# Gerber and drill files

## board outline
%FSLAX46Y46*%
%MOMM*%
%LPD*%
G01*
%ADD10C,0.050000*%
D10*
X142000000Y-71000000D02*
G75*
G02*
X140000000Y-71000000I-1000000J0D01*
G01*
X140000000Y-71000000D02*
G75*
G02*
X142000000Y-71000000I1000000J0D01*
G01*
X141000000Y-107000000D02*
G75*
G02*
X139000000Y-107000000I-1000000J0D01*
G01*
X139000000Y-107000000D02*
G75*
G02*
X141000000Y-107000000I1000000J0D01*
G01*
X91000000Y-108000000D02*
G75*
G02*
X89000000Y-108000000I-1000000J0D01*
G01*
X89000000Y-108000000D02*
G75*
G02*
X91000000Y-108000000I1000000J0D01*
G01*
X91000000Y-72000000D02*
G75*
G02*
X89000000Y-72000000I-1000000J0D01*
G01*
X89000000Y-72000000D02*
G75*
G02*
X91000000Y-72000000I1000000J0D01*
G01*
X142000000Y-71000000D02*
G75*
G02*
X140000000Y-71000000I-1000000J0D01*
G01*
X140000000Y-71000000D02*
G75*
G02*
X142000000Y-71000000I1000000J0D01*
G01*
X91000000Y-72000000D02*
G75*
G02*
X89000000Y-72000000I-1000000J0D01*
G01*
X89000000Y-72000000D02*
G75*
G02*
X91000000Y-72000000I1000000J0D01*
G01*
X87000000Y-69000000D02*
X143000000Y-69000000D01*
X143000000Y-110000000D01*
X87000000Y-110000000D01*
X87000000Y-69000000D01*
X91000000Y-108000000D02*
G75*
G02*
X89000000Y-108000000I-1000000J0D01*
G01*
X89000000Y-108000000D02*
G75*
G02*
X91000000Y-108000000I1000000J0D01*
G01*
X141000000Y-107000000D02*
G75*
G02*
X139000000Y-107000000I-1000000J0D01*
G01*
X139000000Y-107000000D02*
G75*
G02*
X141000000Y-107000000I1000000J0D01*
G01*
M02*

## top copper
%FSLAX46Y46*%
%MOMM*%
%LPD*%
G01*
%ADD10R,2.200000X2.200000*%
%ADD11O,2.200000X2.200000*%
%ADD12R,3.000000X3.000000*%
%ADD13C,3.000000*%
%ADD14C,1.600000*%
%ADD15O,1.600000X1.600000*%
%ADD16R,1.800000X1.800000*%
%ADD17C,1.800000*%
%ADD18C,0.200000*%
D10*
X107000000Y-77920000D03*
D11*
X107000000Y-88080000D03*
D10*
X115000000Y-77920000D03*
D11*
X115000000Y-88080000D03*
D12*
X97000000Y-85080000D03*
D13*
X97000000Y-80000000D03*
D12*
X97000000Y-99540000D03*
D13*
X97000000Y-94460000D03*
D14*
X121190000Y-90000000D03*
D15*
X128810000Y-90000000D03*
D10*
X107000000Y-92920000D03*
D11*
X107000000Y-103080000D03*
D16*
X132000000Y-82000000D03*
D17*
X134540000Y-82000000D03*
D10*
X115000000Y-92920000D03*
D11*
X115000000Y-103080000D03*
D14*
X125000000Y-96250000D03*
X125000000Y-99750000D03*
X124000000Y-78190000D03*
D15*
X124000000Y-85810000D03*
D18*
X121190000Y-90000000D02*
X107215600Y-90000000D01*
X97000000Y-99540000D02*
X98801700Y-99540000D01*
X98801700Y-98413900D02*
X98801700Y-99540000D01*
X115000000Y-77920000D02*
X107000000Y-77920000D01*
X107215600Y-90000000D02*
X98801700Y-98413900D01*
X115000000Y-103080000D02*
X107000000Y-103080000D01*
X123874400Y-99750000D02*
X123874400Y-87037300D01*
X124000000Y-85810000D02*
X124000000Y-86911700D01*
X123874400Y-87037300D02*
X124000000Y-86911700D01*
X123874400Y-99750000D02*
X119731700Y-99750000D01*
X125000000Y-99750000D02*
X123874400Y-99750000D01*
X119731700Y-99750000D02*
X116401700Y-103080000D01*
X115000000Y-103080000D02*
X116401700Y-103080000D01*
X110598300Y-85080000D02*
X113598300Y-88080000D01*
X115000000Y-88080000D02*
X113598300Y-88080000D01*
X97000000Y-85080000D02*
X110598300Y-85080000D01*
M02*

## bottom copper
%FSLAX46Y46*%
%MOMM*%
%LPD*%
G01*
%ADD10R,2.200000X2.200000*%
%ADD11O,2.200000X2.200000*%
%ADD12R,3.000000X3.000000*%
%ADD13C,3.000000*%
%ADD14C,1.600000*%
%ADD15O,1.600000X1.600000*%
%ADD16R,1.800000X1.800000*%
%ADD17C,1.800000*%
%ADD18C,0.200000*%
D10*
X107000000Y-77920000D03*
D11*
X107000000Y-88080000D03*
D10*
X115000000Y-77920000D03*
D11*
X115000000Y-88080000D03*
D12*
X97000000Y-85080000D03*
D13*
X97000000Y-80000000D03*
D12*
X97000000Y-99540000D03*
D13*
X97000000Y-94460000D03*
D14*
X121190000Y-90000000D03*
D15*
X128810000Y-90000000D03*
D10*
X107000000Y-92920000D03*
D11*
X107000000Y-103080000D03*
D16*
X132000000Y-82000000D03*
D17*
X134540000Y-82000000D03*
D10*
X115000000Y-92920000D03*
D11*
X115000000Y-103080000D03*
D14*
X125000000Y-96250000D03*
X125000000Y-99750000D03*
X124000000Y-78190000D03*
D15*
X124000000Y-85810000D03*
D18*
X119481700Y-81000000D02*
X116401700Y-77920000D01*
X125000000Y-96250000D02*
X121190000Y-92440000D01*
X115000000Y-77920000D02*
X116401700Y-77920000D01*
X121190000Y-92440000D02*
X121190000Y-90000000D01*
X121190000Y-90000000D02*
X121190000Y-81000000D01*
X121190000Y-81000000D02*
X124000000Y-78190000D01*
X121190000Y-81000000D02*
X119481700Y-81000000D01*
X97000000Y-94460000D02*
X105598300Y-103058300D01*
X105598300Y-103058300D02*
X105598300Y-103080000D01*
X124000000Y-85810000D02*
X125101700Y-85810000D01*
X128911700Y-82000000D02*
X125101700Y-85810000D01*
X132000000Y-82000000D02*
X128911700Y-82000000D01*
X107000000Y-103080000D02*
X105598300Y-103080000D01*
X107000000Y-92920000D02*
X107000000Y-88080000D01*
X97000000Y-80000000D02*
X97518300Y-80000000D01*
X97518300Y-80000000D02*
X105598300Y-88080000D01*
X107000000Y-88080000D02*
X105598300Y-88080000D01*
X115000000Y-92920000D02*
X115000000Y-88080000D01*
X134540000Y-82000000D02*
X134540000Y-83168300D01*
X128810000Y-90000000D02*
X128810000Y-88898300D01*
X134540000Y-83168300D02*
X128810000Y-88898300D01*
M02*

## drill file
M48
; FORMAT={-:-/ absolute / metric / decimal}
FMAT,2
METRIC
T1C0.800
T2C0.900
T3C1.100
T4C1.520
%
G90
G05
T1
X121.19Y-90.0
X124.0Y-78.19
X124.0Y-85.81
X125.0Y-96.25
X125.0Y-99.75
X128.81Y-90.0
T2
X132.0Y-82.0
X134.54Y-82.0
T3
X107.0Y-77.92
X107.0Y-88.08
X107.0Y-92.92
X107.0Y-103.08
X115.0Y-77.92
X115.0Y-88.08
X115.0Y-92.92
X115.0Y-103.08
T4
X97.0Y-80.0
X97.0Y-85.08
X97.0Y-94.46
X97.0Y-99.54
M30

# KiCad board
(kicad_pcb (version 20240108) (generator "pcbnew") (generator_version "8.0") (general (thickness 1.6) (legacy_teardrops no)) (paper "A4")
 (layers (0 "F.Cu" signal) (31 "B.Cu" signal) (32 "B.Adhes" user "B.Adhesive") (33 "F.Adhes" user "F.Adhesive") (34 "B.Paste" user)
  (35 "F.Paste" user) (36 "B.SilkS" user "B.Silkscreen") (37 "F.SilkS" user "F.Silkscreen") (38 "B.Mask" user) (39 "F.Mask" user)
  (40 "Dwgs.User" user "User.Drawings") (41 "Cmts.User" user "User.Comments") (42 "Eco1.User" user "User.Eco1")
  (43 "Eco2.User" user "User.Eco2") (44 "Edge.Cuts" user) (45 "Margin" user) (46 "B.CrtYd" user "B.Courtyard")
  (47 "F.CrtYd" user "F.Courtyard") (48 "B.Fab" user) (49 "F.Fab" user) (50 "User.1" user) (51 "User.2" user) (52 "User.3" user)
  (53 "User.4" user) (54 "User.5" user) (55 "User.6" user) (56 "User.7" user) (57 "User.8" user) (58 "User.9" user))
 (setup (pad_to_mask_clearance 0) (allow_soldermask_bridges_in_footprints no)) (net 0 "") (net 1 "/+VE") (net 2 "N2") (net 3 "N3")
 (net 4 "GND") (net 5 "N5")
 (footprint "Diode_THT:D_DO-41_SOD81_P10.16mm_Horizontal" (layer "F.Cu") (at 107 77.92 -90)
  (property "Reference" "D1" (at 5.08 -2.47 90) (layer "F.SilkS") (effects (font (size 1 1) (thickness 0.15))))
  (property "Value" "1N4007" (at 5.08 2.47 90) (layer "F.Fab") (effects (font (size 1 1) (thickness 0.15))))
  (pad "1" thru_hole rect (at 0 0 270) (size 2.2 2.2) (drill 1.1) (layers "*.Cu" "*.Mask") (remove_unused_layers no) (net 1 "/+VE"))
  (pad "2" thru_hole oval (at 10.16 0 270) (size 2.2 2.2) (drill 1.1) (layers "*.Cu" "*.Mask") (remove_unused_layers no) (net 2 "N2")))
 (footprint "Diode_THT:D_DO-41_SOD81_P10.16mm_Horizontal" (layer "F.Cu") (at 115 77.92 -90)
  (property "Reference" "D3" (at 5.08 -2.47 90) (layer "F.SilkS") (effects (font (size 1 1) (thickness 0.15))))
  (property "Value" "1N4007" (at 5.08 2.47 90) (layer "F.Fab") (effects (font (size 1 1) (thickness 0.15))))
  (pad "1" thru_hole rect (at 0 0 270) (size 2.2 2.2) (drill 1.1) (layers "*.Cu" "*.Mask") (remove_unused_layers no) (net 1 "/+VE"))
  (pad "2" thru_hole oval (at 10.16 0 270) (size 2.2 2.2) (drill 1.1) (layers "*.Cu" "*.Mask") (remove_unused_layers no) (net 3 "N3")))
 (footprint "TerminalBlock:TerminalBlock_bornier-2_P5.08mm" (layer "F.Cu") (at 97 85.08 90)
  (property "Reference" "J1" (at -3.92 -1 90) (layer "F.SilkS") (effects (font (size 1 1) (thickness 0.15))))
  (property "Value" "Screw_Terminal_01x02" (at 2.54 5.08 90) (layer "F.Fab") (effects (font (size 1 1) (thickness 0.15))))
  (pad "1" thru_hole rect (at 0 0 90) (size 3 3) (drill 1.52) (layers "*.Cu" "*.Mask") (remove_unused_layers no) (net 3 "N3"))
  (pad "2" thru_hole circle (at 5.08 0 90) (size 3 3) (drill 1.52) (layers "*.Cu" "*.Mask") (remove_unused_layers no) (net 2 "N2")))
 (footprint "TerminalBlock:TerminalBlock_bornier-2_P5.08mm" (layer "F.Cu") (at 97 99.54 90)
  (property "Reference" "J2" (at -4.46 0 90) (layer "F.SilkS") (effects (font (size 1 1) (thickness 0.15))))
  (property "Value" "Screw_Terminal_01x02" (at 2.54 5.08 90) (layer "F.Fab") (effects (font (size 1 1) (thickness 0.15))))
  (pad "1" thru_hole rect (at 0 0 90) (size 3 3) (drill 1.52) (layers "*.Cu" "*.Mask") (remove_unused_layers no) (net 1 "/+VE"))
  (pad "2" thru_hole circle (at 5.08 0 90) (size 3 3) (drill 1.52) (layers "*.Cu" "*.Mask") (remove_unused_layers no) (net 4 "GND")))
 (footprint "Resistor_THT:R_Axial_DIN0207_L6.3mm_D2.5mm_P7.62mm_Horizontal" (layer "F.Cu") (at 121.19 90)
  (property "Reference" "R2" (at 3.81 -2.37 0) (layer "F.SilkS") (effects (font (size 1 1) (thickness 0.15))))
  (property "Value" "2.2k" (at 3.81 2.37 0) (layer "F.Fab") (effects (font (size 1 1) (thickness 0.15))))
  (pad "1" thru_hole circle (at 0 0) (size 1.6 1.6) (drill 0.8) (layers "*.Cu" "*.Mask") (remove_unused_layers no) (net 1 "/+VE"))
  (pad "2" thru_hole oval (at 7.62 0) (size 1.6 1.6) (drill 0.8) (layers "*.Cu" "*.Mask") (remove_unused_layers no) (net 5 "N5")))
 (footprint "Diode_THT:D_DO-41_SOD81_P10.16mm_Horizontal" (layer "F.Cu") (at 107 92.92 -90)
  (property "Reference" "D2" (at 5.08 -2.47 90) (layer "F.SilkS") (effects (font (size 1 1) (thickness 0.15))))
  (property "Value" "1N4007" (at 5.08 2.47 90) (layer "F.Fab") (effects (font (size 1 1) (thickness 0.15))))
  (pad "1" thru_hole rect (at 0 0 270) (size 2.2 2.2) (drill 1.1) (layers "*.Cu" "*.Mask") (remove_unused_layers no) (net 2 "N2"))
  (pad "2" thru_hole oval (at 10.16 0 270) (size 2.2 2.2) (drill 1.1) (layers "*.Cu" "*.Mask") (remove_unused_layers no) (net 4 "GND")))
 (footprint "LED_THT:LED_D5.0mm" (layer "F.Cu") (at 132 82)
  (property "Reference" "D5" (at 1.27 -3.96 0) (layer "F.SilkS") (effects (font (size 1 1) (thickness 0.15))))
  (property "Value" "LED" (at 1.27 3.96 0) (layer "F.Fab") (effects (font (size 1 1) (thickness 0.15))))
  (pad "1" thru_hole rect (at 0 0) (size 1.8 1.8) (drill 0.9) (layers "*.Cu" "*.Mask") (remove_unused_layers no) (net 4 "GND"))
  (pad "2" thru_hole circle (at 2.54 0) (size 1.8 1.8) (drill 0.9) (layers "*.Cu" "*.Mask") (remove_unused_layers no) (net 5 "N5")))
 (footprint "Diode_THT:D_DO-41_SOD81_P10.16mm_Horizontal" (layer "F.Cu") (at 115 92.92 -90)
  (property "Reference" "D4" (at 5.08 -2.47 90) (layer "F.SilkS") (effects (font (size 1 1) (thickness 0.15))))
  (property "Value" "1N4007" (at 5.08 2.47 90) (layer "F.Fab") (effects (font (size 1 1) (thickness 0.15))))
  (pad "1" thru_hole rect (at 0 0 270) (size 2.2 2.2) (drill 1.1) (layers "*.Cu" "*.Mask") (remove_unused_layers no) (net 3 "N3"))
  (pad "2" thru_hole oval (at 10.16 0 270) (size 2.2 2.2) (drill 1.1) (layers "*.Cu" "*.Mask") (remove_unused_layers no) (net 4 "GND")))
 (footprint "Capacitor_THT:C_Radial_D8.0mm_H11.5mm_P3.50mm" (layer "F.Cu") (at 125 96.25 -90)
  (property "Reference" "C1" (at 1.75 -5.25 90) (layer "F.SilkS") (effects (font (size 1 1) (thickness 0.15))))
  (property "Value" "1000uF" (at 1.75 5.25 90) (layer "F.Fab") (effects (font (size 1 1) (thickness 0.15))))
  (pad "1" thru_hole circle (at 0 0 270) (size 1.6 1.6) (drill 0.8) (layers "*.Cu" "*.Mask") (remove_unused_layers no) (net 1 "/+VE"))
  (pad "2" thru_hole circle (at 3.5 0 270) (size 1.6 1.6) (drill 0.8) (layers "*.Cu" "*.Mask") (remove_unused_layers no) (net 4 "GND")))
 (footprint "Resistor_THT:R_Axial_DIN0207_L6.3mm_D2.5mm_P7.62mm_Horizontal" (layer "F.Cu") (at 124 78.19 -90)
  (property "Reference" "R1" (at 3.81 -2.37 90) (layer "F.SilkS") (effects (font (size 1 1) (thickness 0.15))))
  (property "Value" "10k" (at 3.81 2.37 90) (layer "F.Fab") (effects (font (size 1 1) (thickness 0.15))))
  (pad "1" thru_hole circle (at 0 0 270) (size 1.6 1.6) (drill 0.8) (layers "*.Cu" "*.Mask") (remove_unused_layers no) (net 1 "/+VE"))
  (pad "2" thru_hole oval (at 7.62 0 270) (size 1.6 1.6) (drill 0.8) (layers "*.Cu" "*.Mask") (remove_unused_layers no) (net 4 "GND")))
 (gr_circle (center 141 71) (end 141 70) (stroke (width 0.05) (type default)) (fill none) (layer "Edge.Cuts"))
 (gr_circle (center 140 107) (end 140 106) (stroke (width 0.05) (type default)) (fill none) (layer "Edge.Cuts"))
 (gr_circle (center 90 108) (end 90 107) (stroke (width 0.05) (type default)) (fill none) (layer "Edge.Cuts"))
 (gr_circle (center 90 72) (end 90 71) (stroke (width 0.05) (type default)) (fill none) (layer "Edge.Cuts"))
 (gr_circle (center 141 71) (end 141 70) (stroke (width 0.05) (type default)) (fill none) (layer "Edge.Cuts"))
 (gr_circle (center 90 72) (end 90 71) (stroke (width 0.05) (type default)) (fill none) (layer "Edge.Cuts"))
 (gr_rect (start 87 69) (end 143 110) (stroke (width 0.05) (type default)) (fill none) (layer "Edge.Cuts"))
 (gr_circle (center 90 108) (end 90 107) (stroke (width 0.05) (type default)) (fill none) (layer "Edge.Cuts"))
 (gr_circle (center 140 107) (end 140 106) (stroke (width 0.05) (type default)) (fill none) (layer "Edge.Cuts"))
 (segment (start 121.19 90) (end 107.2156 90) (width 0.2) (layer "F.Cu") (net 1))
 (segment (start 97 99.54) (end 98.8017 99.54) (width 0.2) (layer "F.Cu") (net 1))
 (segment (start 98.8017 98.4139) (end 98.8017 99.54) (width 0.2) (layer "F.Cu") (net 1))
 (segment (start 115 77.92) (end 107 77.92) (width 0.2) (layer "F.Cu") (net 1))
 (segment (start 107.2156 90) (end 98.8017 98.4139) (width 0.2) (layer "F.Cu") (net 1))
 (segment (start 119.4817 81) (end 116.4017 77.92) (width 0.2) (layer "B.Cu") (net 1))
 (segment (start 125 96.25) (end 121.19 92.44) (width 0.2) (layer "B.Cu") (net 1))
 (segment (start 115 77.92) (end 116.4017 77.92) (width 0.2) (layer "B.Cu") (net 1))
 (segment (start 121.19 92.44) (end 121.19 90) (width 0.2) (layer "B.Cu") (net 1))
 (segment (start 121.19 90) (end 121.19 81) (width 0.2) (layer "B.Cu") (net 1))
 (segment (start 121.19 81) (end 124 78.19) (width 0.2) (layer "B.Cu") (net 1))
 (segment (start 121.19 81) (end 119.4817 81) (width 0.2) (layer "B.Cu") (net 1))
 (segment (start 115 103.08) (end 107 103.08) (width 0.2) (layer "F.Cu") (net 4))
 (segment (start 123.8744 99.75) (end 123.8744 87.0373) (width 0.2) (layer "F.Cu") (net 4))
 (segment (start 124 85.81) (end 124 86.9117) (width 0.2) (layer "F.Cu") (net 4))
 (segment (start 123.8744 87.0373) (end 124 86.9117) (width 0.2) (layer "F.Cu") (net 4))
 (segment (start 123.8744 99.75) (end 119.7317 99.75) (width 0.2) (layer "F.Cu") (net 4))
 (segment (start 125 99.75) (end 123.8744 99.75) (width 0.2) (layer "F.Cu") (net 4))
 (segment (start 119.7317 99.75) (end 116.4017 103.08) (width 0.2) (layer "F.Cu") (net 4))
 (segment (start 115 103.08) (end 116.4017 103.08) (width 0.2) (layer "F.Cu") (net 4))
 (segment (start 97 94.46) (end 105.5983 103.0583) (width 0.2) (layer "B.Cu") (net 4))
 (segment (start 105.5983 103.0583) (end 105.5983 103.08) (width 0.2) (layer "B.Cu") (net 4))
 (segment (start 124 85.81) (end 125.1017 85.81) (width 0.2) (layer "B.Cu") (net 4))
 (segment (start 128.9117 82) (end 125.1017 85.81) (width 0.2) (layer "B.Cu") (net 4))
 (segment (start 132 82) (end 128.9117 82) (width 0.2) (layer "B.Cu") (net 4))
 (segment (start 107 103.08) (end 105.5983 103.08) (width 0.2) (layer "B.Cu") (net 4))
 (segment (start 107 92.92) (end 107 88.08) (width 0.2) (layer "B.Cu") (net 2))
 (segment (start 97 80) (end 97.5183 80) (width 0.2) (layer "B.Cu") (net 2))
 (segment (start 97.5183 80) (end 105.5983 88.08) (width 0.2) (layer "B.Cu") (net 2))
 (segment (start 107 88.08) (end 105.5983 88.08) (width 0.2) (layer "B.Cu") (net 2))
 (segment (start 110.5983 85.08) (end 113.5983 88.08) (width 0.2) (layer "F.Cu") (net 3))
 (segment (start 115 88.08) (end 113.5983 88.08) (width 0.2) (layer "F.Cu") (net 3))
 (segment (start 97 85.08) (end 110.5983 85.08) (width 0.2) (layer "F.Cu") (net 3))
 (segment (start 115 92.92) (end 115 88.08) (width 0.2) (layer "B.Cu") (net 3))
 (segment (start 134.54 82) (end 134.54 83.1683) (width 0.2) (layer "B.Cu") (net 5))
 (segment (start 128.81 90) (end 128.81 88.8983) (width 0.2) (layer "B.Cu") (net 5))
 (segment (start 134.54 83.1683) (end 128.81 88.8983) (width 0.2) (layer "B.Cu") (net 5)))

